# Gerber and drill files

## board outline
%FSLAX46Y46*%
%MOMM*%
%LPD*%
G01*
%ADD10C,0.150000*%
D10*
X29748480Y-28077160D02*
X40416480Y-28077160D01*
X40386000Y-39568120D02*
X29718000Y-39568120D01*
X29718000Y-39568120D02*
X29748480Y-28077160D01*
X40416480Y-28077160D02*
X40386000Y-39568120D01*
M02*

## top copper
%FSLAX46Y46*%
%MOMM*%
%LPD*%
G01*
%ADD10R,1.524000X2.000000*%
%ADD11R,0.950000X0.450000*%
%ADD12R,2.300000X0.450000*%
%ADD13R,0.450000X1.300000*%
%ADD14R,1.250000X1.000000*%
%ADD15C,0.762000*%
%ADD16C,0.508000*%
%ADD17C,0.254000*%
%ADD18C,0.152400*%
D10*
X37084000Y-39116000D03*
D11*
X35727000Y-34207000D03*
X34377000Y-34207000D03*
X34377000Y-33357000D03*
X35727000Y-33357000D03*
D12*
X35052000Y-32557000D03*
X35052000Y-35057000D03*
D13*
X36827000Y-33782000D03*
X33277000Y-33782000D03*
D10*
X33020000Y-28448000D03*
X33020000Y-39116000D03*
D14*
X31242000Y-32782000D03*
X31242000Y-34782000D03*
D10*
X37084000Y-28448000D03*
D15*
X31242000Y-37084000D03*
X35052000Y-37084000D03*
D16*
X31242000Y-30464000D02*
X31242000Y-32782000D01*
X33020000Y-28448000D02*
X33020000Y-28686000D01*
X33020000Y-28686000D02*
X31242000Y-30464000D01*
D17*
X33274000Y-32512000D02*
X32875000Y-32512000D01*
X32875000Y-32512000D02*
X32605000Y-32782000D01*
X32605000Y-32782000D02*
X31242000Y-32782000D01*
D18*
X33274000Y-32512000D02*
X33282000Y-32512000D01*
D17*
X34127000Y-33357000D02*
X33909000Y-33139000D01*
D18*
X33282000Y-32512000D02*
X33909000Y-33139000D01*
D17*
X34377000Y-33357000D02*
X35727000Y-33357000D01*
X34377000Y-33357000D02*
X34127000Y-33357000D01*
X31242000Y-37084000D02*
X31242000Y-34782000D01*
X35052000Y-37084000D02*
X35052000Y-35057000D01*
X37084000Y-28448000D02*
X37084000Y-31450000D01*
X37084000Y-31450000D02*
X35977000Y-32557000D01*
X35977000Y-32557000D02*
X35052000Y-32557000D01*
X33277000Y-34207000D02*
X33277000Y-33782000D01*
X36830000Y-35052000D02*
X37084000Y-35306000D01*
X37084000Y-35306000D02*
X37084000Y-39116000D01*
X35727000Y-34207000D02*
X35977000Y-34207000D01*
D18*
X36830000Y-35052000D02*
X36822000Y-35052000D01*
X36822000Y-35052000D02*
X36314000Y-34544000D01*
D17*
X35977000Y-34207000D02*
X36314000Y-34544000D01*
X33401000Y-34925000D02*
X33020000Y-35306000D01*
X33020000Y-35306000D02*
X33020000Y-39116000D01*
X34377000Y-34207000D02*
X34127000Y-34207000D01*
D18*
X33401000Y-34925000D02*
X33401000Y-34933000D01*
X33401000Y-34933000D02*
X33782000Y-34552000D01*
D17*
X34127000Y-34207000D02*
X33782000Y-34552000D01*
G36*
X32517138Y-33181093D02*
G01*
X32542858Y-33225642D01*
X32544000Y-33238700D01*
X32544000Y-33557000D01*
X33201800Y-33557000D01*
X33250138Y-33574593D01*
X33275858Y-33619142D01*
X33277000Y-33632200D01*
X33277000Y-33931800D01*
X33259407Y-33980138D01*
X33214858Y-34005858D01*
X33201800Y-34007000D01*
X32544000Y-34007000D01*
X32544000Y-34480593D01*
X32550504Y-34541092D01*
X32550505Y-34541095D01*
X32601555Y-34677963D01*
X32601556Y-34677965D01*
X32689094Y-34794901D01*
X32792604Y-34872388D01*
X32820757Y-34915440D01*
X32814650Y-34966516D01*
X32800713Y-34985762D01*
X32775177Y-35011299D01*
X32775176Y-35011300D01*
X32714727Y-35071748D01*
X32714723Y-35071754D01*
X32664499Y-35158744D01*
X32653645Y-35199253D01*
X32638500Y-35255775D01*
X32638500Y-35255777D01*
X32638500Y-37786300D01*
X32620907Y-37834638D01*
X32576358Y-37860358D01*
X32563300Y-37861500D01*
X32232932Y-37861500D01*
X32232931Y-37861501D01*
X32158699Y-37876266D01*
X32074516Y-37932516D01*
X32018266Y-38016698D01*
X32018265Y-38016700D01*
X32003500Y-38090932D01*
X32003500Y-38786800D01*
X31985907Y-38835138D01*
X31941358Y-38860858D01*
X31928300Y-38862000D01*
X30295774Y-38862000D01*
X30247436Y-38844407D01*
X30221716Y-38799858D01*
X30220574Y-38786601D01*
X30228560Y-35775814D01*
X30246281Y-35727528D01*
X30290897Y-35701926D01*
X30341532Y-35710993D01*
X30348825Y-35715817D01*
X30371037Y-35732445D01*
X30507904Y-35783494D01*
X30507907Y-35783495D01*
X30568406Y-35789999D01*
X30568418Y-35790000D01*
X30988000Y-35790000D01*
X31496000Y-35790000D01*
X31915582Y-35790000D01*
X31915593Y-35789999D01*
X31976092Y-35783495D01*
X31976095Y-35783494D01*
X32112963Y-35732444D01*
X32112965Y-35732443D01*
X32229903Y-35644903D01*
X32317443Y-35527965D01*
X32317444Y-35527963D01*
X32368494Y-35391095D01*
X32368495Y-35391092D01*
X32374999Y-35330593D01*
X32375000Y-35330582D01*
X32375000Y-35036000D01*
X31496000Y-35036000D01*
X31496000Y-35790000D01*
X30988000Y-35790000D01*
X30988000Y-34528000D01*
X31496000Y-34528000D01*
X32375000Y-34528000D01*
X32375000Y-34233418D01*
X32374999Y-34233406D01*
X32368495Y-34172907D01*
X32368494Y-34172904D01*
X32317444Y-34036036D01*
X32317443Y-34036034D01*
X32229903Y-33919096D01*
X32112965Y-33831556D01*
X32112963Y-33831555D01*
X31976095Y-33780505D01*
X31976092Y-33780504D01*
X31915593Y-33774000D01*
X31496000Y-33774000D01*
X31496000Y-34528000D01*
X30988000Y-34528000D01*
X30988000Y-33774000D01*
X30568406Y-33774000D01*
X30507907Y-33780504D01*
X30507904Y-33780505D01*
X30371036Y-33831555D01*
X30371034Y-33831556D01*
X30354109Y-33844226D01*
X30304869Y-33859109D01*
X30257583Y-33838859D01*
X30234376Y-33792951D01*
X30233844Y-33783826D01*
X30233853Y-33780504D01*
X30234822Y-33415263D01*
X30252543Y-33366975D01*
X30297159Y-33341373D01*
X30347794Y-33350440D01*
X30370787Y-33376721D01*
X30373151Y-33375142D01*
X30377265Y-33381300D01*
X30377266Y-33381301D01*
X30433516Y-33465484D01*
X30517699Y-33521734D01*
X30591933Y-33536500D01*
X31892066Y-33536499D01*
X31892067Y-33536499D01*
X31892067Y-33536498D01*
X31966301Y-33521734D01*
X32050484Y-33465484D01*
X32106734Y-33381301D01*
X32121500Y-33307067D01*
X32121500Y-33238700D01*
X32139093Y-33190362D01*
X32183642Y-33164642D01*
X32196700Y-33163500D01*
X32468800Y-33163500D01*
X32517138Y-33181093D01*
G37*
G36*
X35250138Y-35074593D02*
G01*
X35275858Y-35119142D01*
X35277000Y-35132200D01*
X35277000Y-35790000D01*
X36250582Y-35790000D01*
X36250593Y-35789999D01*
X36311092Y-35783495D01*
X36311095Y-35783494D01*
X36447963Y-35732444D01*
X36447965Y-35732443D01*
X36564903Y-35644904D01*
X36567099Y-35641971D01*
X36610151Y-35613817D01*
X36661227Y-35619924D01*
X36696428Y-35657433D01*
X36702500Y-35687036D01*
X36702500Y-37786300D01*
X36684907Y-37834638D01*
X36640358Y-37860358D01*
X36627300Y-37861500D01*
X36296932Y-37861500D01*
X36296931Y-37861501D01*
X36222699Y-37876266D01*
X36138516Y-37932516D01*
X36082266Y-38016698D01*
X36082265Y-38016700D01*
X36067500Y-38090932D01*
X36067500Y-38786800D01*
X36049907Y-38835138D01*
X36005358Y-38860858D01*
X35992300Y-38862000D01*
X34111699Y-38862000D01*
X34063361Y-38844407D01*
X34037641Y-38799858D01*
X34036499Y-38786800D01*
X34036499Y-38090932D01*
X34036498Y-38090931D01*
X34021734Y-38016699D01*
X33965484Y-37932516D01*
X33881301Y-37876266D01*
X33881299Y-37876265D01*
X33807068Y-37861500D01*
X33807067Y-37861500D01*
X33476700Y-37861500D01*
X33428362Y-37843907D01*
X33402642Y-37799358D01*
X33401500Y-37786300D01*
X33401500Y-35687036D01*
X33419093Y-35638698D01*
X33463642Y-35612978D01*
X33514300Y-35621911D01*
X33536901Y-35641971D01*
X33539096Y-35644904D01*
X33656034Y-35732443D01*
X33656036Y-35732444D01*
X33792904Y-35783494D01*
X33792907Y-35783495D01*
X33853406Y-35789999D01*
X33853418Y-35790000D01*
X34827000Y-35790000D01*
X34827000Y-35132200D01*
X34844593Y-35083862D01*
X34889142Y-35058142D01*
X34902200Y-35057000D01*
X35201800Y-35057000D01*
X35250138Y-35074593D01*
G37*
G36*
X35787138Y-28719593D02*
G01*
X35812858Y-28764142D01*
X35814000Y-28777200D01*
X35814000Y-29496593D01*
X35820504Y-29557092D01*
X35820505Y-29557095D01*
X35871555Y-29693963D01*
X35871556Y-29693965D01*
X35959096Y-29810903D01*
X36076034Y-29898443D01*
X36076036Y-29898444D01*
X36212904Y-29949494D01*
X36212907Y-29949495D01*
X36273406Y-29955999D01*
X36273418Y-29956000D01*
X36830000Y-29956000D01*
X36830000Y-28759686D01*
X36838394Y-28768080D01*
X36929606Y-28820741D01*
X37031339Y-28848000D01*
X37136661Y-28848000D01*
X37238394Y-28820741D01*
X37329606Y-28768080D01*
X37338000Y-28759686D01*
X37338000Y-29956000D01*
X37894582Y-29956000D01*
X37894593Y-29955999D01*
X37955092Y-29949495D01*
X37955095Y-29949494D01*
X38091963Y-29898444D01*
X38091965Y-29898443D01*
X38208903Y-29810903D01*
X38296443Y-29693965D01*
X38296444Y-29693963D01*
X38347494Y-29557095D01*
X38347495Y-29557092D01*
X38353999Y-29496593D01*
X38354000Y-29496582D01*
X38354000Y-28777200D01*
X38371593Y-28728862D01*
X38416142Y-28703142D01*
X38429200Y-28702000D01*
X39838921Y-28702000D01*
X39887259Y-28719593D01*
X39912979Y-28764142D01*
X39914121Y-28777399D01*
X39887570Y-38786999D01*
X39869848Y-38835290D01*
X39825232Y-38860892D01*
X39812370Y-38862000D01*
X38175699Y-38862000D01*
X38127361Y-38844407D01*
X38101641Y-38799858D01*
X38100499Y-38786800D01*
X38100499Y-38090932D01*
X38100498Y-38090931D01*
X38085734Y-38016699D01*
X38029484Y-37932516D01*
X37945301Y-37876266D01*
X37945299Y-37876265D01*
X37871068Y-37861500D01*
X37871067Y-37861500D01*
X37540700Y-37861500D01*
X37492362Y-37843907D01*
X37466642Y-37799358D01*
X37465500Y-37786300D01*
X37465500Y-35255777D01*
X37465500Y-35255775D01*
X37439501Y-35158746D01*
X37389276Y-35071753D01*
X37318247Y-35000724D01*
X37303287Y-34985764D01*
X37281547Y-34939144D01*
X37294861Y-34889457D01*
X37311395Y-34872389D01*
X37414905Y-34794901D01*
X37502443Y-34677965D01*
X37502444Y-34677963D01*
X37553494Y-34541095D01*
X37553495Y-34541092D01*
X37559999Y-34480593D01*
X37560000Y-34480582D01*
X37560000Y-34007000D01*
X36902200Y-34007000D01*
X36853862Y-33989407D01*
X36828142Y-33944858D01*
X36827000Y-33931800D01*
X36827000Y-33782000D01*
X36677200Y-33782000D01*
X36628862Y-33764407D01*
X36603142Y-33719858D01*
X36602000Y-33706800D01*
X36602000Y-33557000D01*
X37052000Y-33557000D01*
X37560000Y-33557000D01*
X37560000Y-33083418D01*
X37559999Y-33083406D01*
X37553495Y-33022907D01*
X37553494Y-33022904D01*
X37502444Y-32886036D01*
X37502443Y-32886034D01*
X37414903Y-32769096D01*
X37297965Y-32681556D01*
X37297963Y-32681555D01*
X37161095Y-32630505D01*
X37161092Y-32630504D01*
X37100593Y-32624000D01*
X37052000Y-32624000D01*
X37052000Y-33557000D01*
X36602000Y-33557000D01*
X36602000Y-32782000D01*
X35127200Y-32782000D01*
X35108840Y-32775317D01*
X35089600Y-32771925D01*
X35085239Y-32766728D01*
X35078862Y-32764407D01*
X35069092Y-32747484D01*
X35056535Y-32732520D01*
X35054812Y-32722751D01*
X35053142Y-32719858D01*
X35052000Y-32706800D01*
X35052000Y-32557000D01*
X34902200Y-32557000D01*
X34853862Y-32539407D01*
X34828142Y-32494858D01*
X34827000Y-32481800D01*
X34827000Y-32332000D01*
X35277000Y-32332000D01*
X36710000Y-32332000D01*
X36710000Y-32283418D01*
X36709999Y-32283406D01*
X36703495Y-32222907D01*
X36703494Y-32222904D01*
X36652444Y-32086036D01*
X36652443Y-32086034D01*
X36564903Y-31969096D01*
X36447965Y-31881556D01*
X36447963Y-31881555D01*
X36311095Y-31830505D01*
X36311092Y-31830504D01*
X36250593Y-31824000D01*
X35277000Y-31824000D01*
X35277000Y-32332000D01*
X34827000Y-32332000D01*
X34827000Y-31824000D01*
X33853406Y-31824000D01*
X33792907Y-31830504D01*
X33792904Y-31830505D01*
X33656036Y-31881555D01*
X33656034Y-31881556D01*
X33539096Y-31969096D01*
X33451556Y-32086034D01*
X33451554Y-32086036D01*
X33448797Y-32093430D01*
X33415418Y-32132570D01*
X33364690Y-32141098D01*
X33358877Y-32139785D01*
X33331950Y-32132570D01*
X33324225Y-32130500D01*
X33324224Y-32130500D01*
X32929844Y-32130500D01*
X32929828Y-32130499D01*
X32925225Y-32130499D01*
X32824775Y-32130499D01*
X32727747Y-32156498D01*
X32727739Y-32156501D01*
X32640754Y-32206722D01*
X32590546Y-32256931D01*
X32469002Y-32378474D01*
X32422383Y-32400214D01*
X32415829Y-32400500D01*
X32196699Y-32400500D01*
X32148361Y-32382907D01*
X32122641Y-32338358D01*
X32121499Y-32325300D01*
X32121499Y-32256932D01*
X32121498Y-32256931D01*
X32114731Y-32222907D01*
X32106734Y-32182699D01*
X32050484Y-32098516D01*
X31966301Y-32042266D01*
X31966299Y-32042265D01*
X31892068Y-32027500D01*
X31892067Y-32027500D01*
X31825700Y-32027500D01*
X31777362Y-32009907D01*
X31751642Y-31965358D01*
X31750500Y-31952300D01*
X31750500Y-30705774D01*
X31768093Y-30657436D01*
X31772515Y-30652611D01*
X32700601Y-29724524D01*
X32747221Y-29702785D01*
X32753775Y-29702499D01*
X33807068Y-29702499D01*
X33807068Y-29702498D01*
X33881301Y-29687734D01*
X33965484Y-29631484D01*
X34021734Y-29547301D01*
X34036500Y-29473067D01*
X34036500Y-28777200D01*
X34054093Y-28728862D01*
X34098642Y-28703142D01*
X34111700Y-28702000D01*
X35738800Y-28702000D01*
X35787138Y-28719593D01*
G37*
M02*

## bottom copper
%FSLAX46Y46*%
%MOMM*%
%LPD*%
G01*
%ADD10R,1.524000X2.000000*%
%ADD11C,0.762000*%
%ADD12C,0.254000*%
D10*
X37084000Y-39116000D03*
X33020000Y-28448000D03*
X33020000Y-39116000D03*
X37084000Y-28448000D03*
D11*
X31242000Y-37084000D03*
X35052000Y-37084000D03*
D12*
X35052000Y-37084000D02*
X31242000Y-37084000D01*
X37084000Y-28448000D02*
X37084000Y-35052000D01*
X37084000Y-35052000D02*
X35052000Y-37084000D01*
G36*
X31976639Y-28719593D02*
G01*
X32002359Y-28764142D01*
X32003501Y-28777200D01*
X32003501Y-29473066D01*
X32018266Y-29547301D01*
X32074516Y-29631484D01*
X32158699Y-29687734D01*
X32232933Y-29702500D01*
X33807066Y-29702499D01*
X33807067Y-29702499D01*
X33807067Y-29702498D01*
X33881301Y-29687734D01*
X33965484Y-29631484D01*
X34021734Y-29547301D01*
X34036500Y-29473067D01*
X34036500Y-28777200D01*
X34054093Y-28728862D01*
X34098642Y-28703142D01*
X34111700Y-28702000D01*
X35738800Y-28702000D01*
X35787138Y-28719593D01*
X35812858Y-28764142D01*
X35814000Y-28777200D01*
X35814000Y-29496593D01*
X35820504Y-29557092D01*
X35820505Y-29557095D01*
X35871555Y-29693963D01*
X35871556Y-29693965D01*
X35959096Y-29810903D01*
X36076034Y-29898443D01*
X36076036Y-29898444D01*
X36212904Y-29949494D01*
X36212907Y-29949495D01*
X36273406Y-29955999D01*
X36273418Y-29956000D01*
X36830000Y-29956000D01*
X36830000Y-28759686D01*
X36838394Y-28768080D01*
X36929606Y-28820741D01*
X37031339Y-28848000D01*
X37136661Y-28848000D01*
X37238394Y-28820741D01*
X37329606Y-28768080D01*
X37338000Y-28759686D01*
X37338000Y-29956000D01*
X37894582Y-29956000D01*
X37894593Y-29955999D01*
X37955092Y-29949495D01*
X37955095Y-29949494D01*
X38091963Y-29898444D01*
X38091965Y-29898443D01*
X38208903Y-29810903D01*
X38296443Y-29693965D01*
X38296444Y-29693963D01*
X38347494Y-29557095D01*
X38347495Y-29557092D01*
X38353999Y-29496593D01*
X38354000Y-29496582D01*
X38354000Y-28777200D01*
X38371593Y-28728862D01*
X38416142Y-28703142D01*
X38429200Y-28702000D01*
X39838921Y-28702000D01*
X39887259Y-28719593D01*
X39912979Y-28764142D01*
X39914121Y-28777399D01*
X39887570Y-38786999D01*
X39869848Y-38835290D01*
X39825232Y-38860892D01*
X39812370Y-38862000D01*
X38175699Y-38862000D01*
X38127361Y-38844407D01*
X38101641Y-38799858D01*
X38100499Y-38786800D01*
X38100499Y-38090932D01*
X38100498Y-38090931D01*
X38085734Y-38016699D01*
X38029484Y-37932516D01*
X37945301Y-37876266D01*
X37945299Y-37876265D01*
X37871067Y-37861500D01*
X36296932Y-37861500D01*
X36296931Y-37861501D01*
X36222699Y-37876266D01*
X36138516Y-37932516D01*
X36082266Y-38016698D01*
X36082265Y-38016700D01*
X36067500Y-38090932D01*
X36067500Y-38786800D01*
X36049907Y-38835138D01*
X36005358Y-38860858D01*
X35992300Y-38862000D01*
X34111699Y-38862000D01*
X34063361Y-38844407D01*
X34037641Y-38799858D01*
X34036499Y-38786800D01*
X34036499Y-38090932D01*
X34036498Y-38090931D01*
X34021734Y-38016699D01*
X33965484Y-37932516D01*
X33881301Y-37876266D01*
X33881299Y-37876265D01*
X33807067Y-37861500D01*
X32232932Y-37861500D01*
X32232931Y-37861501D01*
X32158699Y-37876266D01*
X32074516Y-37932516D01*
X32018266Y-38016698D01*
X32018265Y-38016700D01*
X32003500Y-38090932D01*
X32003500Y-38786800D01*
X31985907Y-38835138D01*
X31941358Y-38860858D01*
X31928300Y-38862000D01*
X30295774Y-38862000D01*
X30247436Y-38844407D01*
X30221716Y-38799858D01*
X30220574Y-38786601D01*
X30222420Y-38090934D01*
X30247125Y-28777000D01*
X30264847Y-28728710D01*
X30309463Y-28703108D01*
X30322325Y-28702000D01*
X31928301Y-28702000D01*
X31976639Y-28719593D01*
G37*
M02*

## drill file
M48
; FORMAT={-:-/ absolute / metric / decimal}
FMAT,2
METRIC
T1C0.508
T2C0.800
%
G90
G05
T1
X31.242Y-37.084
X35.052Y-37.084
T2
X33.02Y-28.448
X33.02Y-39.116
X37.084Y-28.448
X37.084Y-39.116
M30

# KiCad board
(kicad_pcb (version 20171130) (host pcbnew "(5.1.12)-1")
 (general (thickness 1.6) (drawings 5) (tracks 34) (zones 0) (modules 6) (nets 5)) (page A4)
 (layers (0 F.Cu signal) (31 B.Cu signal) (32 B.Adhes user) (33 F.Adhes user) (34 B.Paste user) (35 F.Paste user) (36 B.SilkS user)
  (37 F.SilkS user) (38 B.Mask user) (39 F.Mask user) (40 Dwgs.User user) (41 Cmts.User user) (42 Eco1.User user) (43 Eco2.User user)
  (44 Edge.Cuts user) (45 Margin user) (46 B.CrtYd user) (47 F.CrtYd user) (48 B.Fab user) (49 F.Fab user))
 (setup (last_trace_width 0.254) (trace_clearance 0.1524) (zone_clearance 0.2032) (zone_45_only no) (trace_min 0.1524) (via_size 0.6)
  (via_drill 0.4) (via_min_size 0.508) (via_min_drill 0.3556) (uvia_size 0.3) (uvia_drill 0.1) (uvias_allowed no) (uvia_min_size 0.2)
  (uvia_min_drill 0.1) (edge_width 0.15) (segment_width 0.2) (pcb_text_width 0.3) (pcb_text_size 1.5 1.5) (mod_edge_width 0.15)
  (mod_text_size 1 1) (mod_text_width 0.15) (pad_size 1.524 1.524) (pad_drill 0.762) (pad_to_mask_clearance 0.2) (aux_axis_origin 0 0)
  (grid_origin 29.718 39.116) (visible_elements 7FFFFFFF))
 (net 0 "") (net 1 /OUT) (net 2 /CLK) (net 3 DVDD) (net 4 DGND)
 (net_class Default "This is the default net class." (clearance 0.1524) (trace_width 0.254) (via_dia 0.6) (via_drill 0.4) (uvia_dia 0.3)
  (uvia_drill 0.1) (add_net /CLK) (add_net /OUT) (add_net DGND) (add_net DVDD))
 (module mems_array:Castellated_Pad (layer F.Cu) (at 37.084 39.116)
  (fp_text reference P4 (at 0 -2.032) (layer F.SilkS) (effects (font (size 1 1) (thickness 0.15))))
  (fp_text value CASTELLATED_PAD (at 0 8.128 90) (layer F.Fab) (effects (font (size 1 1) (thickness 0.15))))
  (pad 1 thru_hole rect (at 0 0) (size 1.524 2) (drill 0.8) (layers *.Cu *.Mask F.SilkS) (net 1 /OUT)))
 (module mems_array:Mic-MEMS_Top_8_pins (layer F.Cu) (at 35.052 33.782 90)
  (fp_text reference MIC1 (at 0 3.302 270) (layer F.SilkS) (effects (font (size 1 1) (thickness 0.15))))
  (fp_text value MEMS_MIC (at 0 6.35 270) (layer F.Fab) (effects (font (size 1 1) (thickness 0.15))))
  (pad 4 smd rect (at -0.425 0.675 90) (size 0.45 0.95) (layers F.Cu F.Paste F.Mask) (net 1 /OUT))
  (pad 3 smd rect (at -0.425 -0.675 90) (size 0.45 0.95) (layers F.Cu F.Paste F.Mask) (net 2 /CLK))
  (pad 2 smd rect (at 0.425 -0.675 90) (size 0.45 0.95) (layers F.Cu F.Paste F.Mask) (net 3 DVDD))
  (pad 1 smd rect (at 0.425 0.675 90) (size 0.45 0.95) (layers F.Cu F.Paste F.Mask) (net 3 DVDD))
  (pad 5 smd rect (at 1.225 0 90) (size 0.45 2.3) (layers F.Cu F.Paste F.Mask) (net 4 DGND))
  (pad 5 smd rect (at -1.275 0 90) (size 0.45 2.3) (layers F.Cu F.Paste F.Mask) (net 4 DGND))
  (pad 5 smd rect (at 0 1.775 90) (size 1.3 0.45) (layers F.Cu F.Paste F.Mask) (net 4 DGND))
  (pad 5 smd rect (at 0 -1.775 90) (size 1.3 0.45) (layers F.Cu F.Paste F.Mask) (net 4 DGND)))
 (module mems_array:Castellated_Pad (layer F.Cu) (at 33.02 28.448)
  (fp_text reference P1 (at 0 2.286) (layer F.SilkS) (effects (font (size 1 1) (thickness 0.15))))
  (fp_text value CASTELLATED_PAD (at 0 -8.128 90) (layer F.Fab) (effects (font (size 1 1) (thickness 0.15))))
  (pad 1 thru_hole rect (at 0 0) (size 1.524 2) (drill 0.8) (layers *.Cu *.Mask F.SilkS) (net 3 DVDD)))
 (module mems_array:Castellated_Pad (layer F.Cu) (at 33.02 39.116)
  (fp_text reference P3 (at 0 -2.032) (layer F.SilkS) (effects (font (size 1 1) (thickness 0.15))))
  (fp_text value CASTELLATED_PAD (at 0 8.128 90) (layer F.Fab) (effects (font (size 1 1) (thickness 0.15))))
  (pad 1 thru_hole rect (at 0 0) (size 1.524 2) (drill 0.8) (layers *.Cu *.Mask F.SilkS) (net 2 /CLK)))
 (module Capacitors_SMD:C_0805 (layer F.Cu) (at 31.242 33.782 270)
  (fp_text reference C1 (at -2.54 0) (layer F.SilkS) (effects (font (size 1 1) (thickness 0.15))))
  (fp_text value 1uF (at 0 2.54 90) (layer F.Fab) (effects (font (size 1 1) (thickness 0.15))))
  (pad 1 smd rect (at -1 0 270) (size 1 1.25) (layers F.Cu F.Paste F.Mask) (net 3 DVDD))
  (pad 2 smd rect (at 1 0 270) (size 1 1.25) (layers F.Cu F.Paste F.Mask) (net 4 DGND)))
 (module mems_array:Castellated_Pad (layer F.Cu) (at 37.084 28.448)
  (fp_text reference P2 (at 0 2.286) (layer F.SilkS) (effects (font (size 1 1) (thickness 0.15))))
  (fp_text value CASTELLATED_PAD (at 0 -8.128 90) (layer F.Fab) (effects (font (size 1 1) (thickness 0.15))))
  (pad 1 thru_hole rect (at 0 0) (size 1.524 2) (drill 0.8) (layers *.Cu *.Mask F.SilkS) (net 4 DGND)))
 (gr_line (start 29.74848 28.07716) (end 40.41648 28.07716) (layer Edge.Cuts) (width 0.15))
 (gr_line (start 40.386 39.56812) (end 29.718 39.56812) (layer Edge.Cuts) (width 0.15))
 (gr_line (start 29.718 39.56812) (end 29.74848 28.07716) (layer Edge.Cuts) (width 0.15))
 (gr_line (start 40.41648 28.07716) (end 40.386 39.56812) (layer Edge.Cuts) (width 0.15))
 (segment (start 31.242 30.464) (end 31.242 32.782) (width 0.508) (layer F.Cu) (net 3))
 (segment (start 33.02 28.448) (end 33.02 28.686) (width 0.508) (layer F.Cu) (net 3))
 (segment (start 33.02 28.686) (end 31.242 30.464) (width 0.508) (layer F.Cu) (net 3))
 (segment (start 33.274 32.512) (end 32.875 32.512) (width 0.254) (layer F.Cu) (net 3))
 (segment (start 32.875 32.512) (end 32.605 32.782) (width 0.254) (layer F.Cu) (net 3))
 (segment (start 32.605 32.782) (end 31.242 32.782) (width 0.254) (layer F.Cu) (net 3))
 (segment (start 33.274 32.512) (end 33.282 32.512) (width 0.1524) (layer F.Cu) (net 3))
 (segment (start 34.127 33.357) (end 33.909 33.139) (width 0.254) (layer F.Cu) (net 3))
 (segment (start 33.282 32.512) (end 33.909 33.139) (width 0.1524) (layer F.Cu) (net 3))
 (segment (start 34.377 33.357) (end 35.727 33.357) (width 0.254) (layer F.Cu) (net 3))
 (segment (start 34.377 33.357) (end 34.127 33.357) (width 0.254) (layer F.Cu) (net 3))
 (segment (start 31.242 37.084) (end 31.242 34.782) (width 0.254) (layer F.Cu) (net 4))
 (segment (start 35.052 37.084) (end 31.242 37.084) (width 0.254) (layer B.Cu) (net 4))
 (via (at 31.242 37.084) (size 0.762) (drill 0.508) (layers F.Cu B.Cu) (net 4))
 (segment (start 35.052 37.084) (end 35.052 35.057) (width 0.254) (layer F.Cu) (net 4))
 (segment (start 37.084 28.448) (end 37.084 35.052) (width 0.254) (layer B.Cu) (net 4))
 (segment (start 37.084 35.052) (end 35.052 37.084) (width 0.254) (layer B.Cu) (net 4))
 (via (at 35.052 37.084) (size 0.762) (drill 0.508) (layers F.Cu B.Cu) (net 4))
 (segment (start 37.084 28.448) (end 37.084 31.45) (width 0.254) (layer F.Cu) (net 4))
 (segment (start 37.084 31.45) (end 35.977 32.557) (width 0.254) (layer F.Cu) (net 4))
 (segment (start 35.977 32.557) (end 35.052 32.557) (width 0.254) (layer F.Cu) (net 4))
 (segment (start 33.277 34.207) (end 33.277 33.782) (width 0.254) (layer F.Cu) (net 4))
 (segment (start 36.83 35.052) (end 37.084 35.306) (width 0.254) (layer F.Cu) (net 1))
 (segment (start 37.084 35.306) (end 37.084 39.116) (width 0.254) (layer F.Cu) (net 1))
 (segment (start 35.727 34.207) (end 35.977 34.207) (width 0.254) (layer F.Cu) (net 1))
 (segment (start 36.83 35.052) (end 36.822 35.052) (width 0.1524) (layer F.Cu) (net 1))
 (segment (start 36.822 35.052) (end 36.314 34.544) (width 0.1524) (layer F.Cu) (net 1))
 (segment (start 35.977 34.207) (end 36.314 34.544) (width 0.254) (layer F.Cu) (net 1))
 (segment (start 33.401 34.925) (end 33.02 35.306) (width 0.254) (layer F.Cu) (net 2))
 (segment (start 33.02 35.306) (end 33.02 39.116) (width 0.254) (layer F.Cu) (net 2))
 (segment (start 34.377 34.207) (end 34.127 34.207) (width 0.254) (layer F.Cu) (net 2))
 (segment (start 33.401 34.925) (end 33.401 34.933) (width 0.1524) (layer F.Cu) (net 2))
 (segment (start 33.401 34.933) (end 33.782 34.552) (width 0.1524) (layer F.Cu) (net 2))
 (segment (start 34.127 34.207) (end 33.782 34.552) (width 0.254) (layer F.Cu) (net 2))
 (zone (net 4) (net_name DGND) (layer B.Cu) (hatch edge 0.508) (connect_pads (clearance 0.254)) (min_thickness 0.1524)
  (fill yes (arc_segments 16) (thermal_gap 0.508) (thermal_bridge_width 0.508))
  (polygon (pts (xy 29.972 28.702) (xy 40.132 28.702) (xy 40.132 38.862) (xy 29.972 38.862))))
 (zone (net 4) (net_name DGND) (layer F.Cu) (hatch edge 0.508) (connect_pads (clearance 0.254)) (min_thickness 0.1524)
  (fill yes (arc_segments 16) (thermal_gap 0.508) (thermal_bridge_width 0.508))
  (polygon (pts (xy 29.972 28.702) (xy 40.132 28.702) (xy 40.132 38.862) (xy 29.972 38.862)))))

